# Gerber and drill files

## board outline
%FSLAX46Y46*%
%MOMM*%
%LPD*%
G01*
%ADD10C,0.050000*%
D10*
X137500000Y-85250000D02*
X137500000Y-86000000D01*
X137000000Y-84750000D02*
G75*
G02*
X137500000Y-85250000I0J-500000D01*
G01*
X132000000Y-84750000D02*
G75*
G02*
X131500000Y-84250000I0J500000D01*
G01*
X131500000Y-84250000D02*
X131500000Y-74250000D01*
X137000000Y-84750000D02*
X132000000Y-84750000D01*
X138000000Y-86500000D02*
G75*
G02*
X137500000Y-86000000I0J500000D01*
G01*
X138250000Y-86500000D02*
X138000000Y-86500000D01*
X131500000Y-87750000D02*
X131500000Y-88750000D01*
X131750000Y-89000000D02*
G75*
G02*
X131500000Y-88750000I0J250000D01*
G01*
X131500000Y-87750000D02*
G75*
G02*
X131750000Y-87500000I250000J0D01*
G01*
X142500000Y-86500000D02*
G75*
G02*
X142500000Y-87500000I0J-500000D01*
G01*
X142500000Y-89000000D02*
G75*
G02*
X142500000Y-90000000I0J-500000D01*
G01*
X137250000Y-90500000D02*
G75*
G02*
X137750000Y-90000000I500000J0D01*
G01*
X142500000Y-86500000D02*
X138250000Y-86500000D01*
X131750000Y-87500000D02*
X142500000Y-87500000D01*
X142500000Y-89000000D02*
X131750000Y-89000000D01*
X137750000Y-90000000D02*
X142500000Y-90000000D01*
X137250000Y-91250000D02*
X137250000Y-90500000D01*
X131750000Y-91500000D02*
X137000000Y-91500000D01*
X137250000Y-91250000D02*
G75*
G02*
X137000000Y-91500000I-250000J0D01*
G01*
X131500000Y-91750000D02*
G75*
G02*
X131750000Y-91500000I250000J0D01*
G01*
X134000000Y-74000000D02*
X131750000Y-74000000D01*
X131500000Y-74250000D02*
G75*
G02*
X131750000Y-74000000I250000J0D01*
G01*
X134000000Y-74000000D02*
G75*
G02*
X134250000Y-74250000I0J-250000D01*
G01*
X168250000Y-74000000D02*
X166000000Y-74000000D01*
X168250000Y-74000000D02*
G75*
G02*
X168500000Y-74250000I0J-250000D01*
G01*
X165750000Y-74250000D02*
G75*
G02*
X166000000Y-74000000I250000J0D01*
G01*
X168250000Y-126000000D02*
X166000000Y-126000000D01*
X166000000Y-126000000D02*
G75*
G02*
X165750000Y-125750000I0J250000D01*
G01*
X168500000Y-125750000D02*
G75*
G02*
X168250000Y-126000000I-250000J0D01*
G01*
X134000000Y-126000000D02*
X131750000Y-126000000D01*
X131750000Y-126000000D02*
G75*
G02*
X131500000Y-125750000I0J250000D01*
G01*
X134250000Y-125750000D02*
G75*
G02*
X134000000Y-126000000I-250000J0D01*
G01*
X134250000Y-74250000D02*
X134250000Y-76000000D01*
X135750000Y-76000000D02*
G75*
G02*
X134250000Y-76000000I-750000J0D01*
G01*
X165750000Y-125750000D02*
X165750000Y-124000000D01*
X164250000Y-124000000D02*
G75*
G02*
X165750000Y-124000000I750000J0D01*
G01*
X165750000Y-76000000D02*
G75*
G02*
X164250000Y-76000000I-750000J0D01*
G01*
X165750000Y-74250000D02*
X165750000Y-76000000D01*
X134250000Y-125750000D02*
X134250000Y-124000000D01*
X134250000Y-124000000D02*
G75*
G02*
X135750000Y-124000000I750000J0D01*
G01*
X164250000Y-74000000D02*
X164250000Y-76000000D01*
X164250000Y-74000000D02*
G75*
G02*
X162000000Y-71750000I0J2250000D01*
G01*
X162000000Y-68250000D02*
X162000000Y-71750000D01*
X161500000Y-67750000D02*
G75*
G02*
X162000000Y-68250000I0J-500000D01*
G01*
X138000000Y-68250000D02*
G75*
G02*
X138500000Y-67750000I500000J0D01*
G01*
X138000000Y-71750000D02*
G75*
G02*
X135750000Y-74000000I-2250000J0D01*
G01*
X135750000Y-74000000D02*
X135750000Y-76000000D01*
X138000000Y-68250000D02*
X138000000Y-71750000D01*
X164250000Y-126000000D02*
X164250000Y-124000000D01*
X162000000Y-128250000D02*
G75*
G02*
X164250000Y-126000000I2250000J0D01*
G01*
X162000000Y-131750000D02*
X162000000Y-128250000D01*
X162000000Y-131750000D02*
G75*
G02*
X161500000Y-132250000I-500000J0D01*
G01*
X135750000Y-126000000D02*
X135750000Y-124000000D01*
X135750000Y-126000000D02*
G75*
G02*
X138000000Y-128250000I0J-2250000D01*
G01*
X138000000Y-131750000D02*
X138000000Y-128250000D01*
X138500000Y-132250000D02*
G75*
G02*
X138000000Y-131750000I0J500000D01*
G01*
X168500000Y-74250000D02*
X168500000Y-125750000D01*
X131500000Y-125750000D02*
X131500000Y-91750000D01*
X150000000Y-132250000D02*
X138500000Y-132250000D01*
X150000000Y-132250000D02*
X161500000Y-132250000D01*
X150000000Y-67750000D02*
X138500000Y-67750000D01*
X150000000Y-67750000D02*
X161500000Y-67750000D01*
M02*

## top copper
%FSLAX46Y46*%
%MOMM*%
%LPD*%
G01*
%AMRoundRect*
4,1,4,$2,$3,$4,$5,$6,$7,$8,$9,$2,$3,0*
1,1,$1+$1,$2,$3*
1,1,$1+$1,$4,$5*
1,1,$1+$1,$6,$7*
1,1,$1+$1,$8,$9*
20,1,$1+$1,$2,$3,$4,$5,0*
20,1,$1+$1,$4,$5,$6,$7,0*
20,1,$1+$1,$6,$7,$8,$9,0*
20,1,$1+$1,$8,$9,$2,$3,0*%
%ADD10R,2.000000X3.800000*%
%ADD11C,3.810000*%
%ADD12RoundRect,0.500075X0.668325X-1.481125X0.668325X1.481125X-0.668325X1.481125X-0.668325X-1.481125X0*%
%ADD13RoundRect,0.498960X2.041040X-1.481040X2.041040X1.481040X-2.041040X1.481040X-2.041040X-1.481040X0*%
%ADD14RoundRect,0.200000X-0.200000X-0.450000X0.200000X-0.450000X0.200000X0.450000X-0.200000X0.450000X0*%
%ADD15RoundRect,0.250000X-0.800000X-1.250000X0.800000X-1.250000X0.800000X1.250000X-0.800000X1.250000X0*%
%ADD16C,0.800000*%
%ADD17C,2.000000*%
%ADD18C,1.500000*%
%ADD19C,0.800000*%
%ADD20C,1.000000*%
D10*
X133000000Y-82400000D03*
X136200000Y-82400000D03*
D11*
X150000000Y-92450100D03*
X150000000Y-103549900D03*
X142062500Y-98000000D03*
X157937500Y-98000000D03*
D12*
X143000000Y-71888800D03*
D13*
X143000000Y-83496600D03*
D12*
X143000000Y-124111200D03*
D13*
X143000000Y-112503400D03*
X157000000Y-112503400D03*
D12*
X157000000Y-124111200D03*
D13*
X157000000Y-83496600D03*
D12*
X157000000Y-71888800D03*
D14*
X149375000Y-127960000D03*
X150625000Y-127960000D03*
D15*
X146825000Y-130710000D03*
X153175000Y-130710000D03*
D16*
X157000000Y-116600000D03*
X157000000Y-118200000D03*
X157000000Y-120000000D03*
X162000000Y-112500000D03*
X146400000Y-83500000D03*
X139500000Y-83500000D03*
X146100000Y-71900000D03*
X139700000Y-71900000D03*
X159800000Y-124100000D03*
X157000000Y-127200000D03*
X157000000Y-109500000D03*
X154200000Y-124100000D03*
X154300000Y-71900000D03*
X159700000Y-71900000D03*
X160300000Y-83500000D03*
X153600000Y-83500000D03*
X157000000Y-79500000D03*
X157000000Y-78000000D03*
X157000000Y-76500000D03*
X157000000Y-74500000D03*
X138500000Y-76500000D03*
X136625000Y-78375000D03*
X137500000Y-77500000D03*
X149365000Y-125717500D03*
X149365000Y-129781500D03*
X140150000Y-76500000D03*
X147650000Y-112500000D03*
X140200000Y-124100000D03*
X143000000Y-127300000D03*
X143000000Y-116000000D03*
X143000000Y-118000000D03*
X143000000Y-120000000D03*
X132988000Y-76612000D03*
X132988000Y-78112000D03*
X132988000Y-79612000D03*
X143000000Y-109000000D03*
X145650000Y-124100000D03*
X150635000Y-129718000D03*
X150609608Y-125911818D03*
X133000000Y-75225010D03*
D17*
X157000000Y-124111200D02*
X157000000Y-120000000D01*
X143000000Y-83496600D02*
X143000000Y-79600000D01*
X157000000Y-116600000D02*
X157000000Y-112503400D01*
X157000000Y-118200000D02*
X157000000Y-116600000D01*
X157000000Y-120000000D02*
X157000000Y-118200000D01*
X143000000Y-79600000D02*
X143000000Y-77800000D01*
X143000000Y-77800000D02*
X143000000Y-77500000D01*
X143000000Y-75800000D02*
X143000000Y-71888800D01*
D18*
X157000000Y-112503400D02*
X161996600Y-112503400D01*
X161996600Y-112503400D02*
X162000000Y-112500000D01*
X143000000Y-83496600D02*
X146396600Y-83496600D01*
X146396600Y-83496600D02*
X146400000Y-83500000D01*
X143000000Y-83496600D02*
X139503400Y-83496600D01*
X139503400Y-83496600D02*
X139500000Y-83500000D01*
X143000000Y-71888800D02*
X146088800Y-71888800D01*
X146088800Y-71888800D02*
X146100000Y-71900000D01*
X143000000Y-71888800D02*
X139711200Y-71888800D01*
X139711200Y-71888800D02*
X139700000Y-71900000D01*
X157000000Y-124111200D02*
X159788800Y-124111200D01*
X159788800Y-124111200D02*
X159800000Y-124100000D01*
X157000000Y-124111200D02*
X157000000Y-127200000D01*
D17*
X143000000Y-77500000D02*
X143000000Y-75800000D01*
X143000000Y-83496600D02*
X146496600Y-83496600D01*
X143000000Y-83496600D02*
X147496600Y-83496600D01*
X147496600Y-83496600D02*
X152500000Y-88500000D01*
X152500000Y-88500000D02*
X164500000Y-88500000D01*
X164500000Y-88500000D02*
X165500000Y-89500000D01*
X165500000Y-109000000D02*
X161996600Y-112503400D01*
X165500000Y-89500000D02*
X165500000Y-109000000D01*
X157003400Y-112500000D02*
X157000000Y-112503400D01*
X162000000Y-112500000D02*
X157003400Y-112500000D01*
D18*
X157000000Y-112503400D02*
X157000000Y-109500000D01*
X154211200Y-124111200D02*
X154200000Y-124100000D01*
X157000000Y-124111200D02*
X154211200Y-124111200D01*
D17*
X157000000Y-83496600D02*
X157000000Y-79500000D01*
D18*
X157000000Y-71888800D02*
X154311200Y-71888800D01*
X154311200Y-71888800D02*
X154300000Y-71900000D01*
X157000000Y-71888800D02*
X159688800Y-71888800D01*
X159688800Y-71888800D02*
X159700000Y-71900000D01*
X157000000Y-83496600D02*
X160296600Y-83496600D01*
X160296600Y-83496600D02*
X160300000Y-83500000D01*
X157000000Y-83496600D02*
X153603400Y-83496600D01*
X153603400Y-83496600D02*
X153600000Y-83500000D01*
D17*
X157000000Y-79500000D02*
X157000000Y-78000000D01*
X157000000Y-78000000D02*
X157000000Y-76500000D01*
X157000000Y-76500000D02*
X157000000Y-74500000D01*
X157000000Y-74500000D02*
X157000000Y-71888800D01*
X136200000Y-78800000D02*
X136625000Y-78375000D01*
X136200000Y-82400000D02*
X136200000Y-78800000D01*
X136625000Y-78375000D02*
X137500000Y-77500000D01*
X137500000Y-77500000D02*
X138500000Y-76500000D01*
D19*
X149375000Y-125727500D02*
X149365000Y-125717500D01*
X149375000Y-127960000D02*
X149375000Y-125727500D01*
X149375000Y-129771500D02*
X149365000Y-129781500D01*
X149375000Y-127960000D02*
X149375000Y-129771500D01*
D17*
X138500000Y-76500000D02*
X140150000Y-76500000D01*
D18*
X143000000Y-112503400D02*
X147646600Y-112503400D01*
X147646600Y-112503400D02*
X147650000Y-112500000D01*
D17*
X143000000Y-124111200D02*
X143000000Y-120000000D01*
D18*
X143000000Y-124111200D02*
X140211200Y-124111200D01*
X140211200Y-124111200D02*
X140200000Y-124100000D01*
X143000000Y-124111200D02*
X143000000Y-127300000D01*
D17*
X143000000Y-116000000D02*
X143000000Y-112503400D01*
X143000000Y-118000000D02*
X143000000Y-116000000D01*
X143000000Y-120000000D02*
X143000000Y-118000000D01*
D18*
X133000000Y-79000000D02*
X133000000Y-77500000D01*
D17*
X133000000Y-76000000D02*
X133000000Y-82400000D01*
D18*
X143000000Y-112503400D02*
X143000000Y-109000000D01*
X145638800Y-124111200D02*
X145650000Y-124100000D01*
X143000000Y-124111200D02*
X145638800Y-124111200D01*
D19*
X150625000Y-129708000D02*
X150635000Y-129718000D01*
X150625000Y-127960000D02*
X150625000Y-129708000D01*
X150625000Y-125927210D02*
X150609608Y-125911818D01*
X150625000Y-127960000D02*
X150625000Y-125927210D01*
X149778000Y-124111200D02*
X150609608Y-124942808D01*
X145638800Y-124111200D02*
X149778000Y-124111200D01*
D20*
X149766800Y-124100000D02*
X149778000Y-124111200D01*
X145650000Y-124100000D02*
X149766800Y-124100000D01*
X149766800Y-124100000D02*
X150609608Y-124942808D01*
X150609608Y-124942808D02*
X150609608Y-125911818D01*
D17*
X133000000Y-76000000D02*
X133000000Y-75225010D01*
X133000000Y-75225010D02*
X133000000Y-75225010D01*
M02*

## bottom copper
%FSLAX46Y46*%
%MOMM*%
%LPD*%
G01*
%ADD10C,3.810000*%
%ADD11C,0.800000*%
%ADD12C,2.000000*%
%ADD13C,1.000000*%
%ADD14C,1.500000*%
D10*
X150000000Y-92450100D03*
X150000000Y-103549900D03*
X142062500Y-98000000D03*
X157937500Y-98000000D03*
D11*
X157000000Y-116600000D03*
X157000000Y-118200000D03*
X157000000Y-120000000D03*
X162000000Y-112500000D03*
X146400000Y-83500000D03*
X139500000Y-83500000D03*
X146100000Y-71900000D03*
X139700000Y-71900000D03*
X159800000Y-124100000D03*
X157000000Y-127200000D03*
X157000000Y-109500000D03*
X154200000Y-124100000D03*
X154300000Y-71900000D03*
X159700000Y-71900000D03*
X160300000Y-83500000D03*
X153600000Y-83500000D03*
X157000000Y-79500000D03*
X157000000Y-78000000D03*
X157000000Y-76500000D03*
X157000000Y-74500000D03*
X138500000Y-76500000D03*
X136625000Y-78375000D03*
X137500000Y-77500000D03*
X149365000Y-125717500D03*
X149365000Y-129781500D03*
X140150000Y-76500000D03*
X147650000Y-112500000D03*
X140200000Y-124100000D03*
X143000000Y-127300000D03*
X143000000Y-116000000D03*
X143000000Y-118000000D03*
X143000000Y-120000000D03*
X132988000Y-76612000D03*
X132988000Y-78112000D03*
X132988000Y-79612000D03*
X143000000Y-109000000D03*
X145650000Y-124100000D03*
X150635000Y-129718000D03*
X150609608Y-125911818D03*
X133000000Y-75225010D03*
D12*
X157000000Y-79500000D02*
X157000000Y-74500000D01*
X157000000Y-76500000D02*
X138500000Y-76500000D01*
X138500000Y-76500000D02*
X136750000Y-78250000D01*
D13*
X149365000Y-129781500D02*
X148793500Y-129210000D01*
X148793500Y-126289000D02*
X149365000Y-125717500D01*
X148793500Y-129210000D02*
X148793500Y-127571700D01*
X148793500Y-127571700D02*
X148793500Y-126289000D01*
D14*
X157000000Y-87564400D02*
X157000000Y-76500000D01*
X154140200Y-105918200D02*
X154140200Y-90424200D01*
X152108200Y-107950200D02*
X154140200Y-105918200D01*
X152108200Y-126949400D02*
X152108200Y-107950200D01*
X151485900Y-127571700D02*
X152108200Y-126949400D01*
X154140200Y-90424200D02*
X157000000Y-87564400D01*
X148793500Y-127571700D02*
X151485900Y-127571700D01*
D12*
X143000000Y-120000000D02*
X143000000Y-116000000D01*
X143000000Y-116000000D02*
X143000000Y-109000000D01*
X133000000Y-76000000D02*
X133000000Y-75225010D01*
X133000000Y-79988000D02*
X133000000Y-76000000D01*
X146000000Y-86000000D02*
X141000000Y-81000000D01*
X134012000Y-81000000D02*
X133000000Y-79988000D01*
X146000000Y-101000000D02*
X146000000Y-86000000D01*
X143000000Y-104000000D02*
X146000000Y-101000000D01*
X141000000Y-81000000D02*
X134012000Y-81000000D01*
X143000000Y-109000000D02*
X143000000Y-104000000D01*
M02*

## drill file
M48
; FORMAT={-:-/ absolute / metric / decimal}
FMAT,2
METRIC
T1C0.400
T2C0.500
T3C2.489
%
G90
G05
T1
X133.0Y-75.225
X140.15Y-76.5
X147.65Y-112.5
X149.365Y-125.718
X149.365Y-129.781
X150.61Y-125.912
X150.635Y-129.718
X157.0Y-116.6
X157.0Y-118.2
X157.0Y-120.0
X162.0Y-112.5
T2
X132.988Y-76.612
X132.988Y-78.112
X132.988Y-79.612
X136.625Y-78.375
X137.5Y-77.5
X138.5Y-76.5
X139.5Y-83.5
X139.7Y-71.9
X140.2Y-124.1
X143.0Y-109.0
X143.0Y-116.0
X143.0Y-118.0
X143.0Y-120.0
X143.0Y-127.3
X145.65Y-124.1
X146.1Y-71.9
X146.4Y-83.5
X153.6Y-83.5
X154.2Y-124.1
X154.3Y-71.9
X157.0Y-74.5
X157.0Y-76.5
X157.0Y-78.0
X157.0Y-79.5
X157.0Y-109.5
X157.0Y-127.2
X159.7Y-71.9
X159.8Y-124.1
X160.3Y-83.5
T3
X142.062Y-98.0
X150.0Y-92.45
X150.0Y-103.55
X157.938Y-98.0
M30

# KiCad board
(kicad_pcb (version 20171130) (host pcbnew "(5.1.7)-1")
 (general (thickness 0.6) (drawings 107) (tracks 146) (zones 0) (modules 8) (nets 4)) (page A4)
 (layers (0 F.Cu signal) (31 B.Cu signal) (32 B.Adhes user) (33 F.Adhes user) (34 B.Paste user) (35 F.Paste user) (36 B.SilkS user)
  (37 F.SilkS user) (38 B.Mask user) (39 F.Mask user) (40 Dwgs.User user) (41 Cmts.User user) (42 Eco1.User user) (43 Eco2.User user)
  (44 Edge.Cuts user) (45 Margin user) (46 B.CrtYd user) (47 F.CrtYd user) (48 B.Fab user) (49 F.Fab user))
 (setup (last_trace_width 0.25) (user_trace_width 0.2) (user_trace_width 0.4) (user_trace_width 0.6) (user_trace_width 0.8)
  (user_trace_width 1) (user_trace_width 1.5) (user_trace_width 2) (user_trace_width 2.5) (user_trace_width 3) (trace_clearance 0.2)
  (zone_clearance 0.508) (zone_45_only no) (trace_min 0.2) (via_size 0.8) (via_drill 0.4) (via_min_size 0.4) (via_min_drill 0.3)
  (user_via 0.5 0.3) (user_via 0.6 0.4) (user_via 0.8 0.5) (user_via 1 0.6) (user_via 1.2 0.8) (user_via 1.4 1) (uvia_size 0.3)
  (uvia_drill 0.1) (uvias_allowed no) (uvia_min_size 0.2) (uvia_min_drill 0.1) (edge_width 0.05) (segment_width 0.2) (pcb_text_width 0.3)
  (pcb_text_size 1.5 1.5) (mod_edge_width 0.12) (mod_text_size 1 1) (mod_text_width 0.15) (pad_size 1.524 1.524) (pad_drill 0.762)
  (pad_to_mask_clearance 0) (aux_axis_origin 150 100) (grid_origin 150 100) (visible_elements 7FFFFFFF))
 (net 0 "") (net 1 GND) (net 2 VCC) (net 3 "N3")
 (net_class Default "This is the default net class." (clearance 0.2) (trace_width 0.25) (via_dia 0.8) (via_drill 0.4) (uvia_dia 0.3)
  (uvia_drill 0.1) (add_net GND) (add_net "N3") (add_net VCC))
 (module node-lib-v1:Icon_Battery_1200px (layer F.Cu) (at 165.1 117.75)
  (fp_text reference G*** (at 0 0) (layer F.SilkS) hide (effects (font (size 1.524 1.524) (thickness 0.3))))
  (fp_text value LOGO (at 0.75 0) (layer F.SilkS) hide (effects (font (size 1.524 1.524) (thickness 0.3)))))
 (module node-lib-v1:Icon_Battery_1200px (layer F.Cu) (at 135.05 117.6)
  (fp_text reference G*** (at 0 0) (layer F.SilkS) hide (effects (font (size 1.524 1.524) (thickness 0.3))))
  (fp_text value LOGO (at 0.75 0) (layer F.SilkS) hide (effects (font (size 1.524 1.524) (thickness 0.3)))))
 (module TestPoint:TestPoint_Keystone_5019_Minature (layer F.Cu) (at 133 82.4 270)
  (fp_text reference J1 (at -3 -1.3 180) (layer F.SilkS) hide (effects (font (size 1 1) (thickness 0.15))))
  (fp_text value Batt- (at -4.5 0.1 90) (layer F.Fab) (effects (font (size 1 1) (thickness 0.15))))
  (pad 1 smd rect (at 0 0 270) (size 3.8 2) (layers F.Cu F.Paste F.Mask) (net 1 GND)))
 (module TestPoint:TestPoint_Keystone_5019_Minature (layer F.Cu) (at 136.2 82.4 90)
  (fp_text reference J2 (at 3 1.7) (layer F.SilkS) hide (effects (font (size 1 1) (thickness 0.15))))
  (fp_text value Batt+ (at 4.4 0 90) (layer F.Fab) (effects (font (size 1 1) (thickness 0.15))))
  (pad 1 smd rect (at 0 0 90) (size 3.8 2) (layers F.Cu F.Paste F.Mask) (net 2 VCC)))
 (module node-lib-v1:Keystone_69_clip (layer F.Cu) (at 150 98 180)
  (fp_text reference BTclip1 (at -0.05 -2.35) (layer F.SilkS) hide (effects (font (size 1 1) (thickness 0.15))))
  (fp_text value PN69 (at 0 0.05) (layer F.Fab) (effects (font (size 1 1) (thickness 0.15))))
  (pad 2 smd circle (at 7.9375 0 180) (size 3.81 3.81) (layers F.Paste F.Mask))
  (pad 2 smd circle (at -7.9375 0 180) (size 3.81 3.81) (layers F.Paste F.Mask))
  (pad 2 smd circle (at 0 -5.5499 180) (size 3.81 3.81) (layers F.Paste F.Mask))
  (pad 2 smd circle (at 0 5.5499 180) (size 3.81 3.81) (layers F.Paste F.Mask))
  (pad 1 thru_hole circle (at 0 5.5499 180) (size 3.81 3.81) (drill 2.4892) (layers *.Cu *.Mask))
  (pad 1 thru_hole circle (at 0 -5.5499 180) (size 3.81 3.81) (drill 2.4892) (layers *.Cu *.Mask))
  (pad 1 thru_hole circle (at 7.9375 0 180) (size 3.81 3.81) (drill 2.4892) (layers *.Cu *.Mask))
  (pad 1 thru_hole circle (at -7.9375 0 180) (size 3.81 3.81) (drill 2.4892) (layers *.Cu *.Mask F.Paste)))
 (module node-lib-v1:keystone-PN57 (layer F.Cu) (at 143 98 90)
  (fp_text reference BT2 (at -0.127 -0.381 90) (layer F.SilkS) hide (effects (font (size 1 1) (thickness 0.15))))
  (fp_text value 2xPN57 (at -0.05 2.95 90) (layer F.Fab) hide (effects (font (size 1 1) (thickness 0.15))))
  (pad 1 smd roundrect (at 26.1112 0 90) (size 3.9624 2.3368) (layers F.Cu F.Paste F.Mask) (roundrect_rratio 0.2139999144128723)
   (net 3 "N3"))
  (pad 1 smd roundrect (at 14.5034 0 90) (size 3.96 5.08) (layers F.Cu F.Paste F.Mask) (roundrect_rratio 0.126) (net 3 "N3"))
  (pad 2 smd roundrect (at -26.1112 0 90) (size 3.9624 2.3368) (layers F.Cu F.Paste F.Mask) (roundrect_rratio 0.2139999144128723)
   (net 1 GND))
  (pad 2 smd roundrect (at -14.5034 0 90) (size 3.96 5.08) (layers F.Cu F.Paste F.Mask) (roundrect_rratio 0.126) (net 1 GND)))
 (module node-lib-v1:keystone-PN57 (layer F.Cu) (at 157 98 90)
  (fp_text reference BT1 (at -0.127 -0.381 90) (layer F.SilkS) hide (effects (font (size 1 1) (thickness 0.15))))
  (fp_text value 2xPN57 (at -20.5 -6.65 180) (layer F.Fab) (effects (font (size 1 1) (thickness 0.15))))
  (pad 2 smd roundrect (at -14.5034 0 90) (size 3.96 5.08) (layers F.Cu F.Paste F.Mask) (roundrect_rratio 0.126) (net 3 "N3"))
  (pad 2 smd roundrect (at -26.1112 0 90) (size 3.9624 2.3368) (layers F.Cu F.Paste F.Mask) (roundrect_rratio 0.2139999144128723)
   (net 3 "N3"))
  (pad 1 smd roundrect (at 14.5034 0 90) (size 3.96 5.08) (layers F.Cu F.Paste F.Mask) (roundrect_rratio 0.126) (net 2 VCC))
  (pad 1 smd roundrect (at 26.1112 0 90) (size 3.9624 2.3368) (layers F.Cu F.Paste F.Mask) (roundrect_rratio 0.2139999144128723) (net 2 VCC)))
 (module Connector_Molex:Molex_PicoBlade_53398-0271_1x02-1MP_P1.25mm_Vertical (layer F.Cu) (at 150 129.21)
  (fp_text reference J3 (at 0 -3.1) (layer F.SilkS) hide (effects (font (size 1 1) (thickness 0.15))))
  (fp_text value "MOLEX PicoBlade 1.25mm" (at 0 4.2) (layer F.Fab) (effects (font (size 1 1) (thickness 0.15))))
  (pad 1 smd roundrect (at -0.625 -1.25) (size 0.8 1.3) (layers F.Cu F.Paste F.Mask) (roundrect_rratio 0.25) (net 2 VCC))
  (pad 2 smd roundrect (at 0.625 -1.25) (size 0.8 1.3) (layers F.Cu F.Paste F.Mask) (roundrect_rratio 0.25) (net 1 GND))
  (pad MP smd roundrect (at -3.175 1.5) (size 2.1 3) (layers F.Cu F.Paste F.Mask) (roundrect_rratio 0.119047619047619))
  (pad MP smd roundrect (at 3.175 1.5) (size 2.1 3) (layers F.Cu F.Paste F.Mask) (roundrect_rratio 0.119047619047619)))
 (gr_line (start 137.5 85.25) (end 137.5 86) (layer Edge.Cuts) (width 0.05))
 (gr_arc (start 137 85.25) (end 137.5 85.25) (angle -90) (layer Edge.Cuts) (width 0.05))
 (gr_arc (start 132 84.25) (end 131.5 84.25) (angle -90) (layer Edge.Cuts) (width 0.05))
 (gr_line (start 131.5 84.25) (end 131.5 74.25) (layer Edge.Cuts) (width 0.05))
 (gr_line (start 137 84.75) (end 132 84.75) (layer Edge.Cuts) (width 0.05))
 (gr_arc (start 138 86) (end 137.5 86) (angle -90) (layer Edge.Cuts) (width 0.05))
 (gr_line (start 138.25 86.5) (end 138 86.5) (layer Edge.Cuts) (width 0.05))
 (gr_line (start 131.5 87.75) (end 131.5 88.75) (layer Edge.Cuts) (width 0.05))
 (gr_arc (start 131.75 88.75) (end 131.5 88.75) (angle -90) (layer Edge.Cuts) (width 0.05))
 (gr_arc (start 131.75 87.75) (end 131.75 87.5) (angle -90) (layer Edge.Cuts) (width 0.05))
 (gr_arc (start 142.5 87) (end 142.5 87.5) (angle -180) (layer Edge.Cuts) (width 0.05))
 (gr_arc (start 142.5 89.5) (end 142.5 90) (angle -180) (layer Edge.Cuts) (width 0.05))
 (gr_arc (start 137.75 90.5) (end 137.75 90) (angle -90) (layer Edge.Cuts) (width 0.05))
 (gr_line (start 142.5 86.5) (end 138.25 86.5) (layer Edge.Cuts) (width 0.05))
 (gr_line (start 131.75 87.5) (end 142.5 87.5) (layer Edge.Cuts) (width 0.05))
 (gr_line (start 142.5 89) (end 131.75 89) (layer Edge.Cuts) (width 0.05))
 (gr_line (start 137.75 90) (end 142.5 90) (layer Edge.Cuts) (width 0.05))
 (gr_line (start 137.25 91.25) (end 137.25 90.5) (layer Edge.Cuts) (width 0.05))
 (gr_line (start 131.75 91.5) (end 137 91.5) (layer Edge.Cuts) (width 0.05))
 (gr_arc (start 137 91.25) (end 137 91.5) (angle -90) (layer Edge.Cuts) (width 0.05))
 (gr_arc (start 131.75 91.75) (end 131.75 91.5) (angle -90) (layer Edge.Cuts) (width 0.05))
 (gr_line (start 134 74) (end 131.75 74) (layer Edge.Cuts) (width 0.05))
 (gr_arc (start 131.75 74.25) (end 131.75 74) (angle -90) (layer Edge.Cuts) (width 0.05))
 (gr_arc (start 134 74.25) (end 134.25 74.25) (angle -90) (layer Edge.Cuts) (width 0.05))
 (gr_line (start 168.25 74) (end 166 74) (layer Edge.Cuts) (width 0.05))
 (gr_arc (start 168.25 74.25) (end 168.5 74.25) (angle -90) (layer Edge.Cuts) (width 0.05))
 (gr_arc (start 166 74.25) (end 166 74) (angle -90) (layer Edge.Cuts) (width 0.05))
 (gr_line (start 168.25 126) (end 166 126) (layer Edge.Cuts) (width 0.05))
 (gr_arc (start 166 125.75) (end 165.75 125.75) (angle -90) (layer Edge.Cuts) (width 0.05))
 (gr_arc (start 168.25 125.75) (end 168.25 126) (angle -90) (layer Edge.Cuts) (width 0.05))
 (gr_line (start 134 126) (end 131.75 126) (layer Edge.Cuts) (width 0.05))
 (gr_arc (start 131.75 125.75) (end 131.5 125.75) (angle -90) (layer Edge.Cuts) (width 0.05))
 (gr_arc (start 134 125.75) (end 134 126) (angle -90) (layer Edge.Cuts) (width 0.05))
 (gr_line (start 134.25 74.25) (end 134.25 76) (layer Edge.Cuts) (width 0.05))
 (gr_arc (start 135 76) (end 134.25 76) (angle -180) (layer Edge.Cuts) (width 0.05))
 (gr_line (start 165.75 125.75) (end 165.75 124) (layer Edge.Cuts) (width 0.05))
 (gr_arc (start 165 124) (end 165.75 124) (angle -180) (layer Edge.Cuts) (width 0.05))
 (gr_arc (start 165 76) (end 164.25 76) (angle -180) (layer Edge.Cuts) (width 0.05))
 (gr_line (start 165.75 74.25) (end 165.75 76) (layer Edge.Cuts) (width 0.05))
 (gr_line (start 134.25 125.75) (end 134.25 124) (layer Edge.Cuts) (width 0.05))
 (gr_arc (start 135 124) (end 135.75 124) (angle -180) (layer Edge.Cuts) (width 0.05))
 (gr_line (start 164.25 74) (end 164.25 76) (layer Edge.Cuts) (width 0.05))
 (gr_arc (start 164.25 71.75) (end 162 71.75) (angle -90) (layer Edge.Cuts) (width 0.05))
 (gr_line (start 162 68.25) (end 162 71.75) (layer Edge.Cuts) (width 0.05))
 (gr_arc (start 161.5 68.25) (end 162 68.25) (angle -90) (layer Edge.Cuts) (width 0.05))
 (gr_arc (start 138.5 68.25) (end 138.5 67.75) (angle -90) (layer Edge.Cuts) (width 0.05))
 (gr_arc (start 135.75 71.75) (end 135.75 74) (angle -90) (layer Edge.Cuts) (width 0.05))
 (gr_line (start 135.75 74) (end 135.75 76) (layer Edge.Cuts) (width 0.05))
 (gr_line (start 138 68.25) (end 138 71.75) (layer Edge.Cuts) (width 0.05))
 (gr_line (start 164.25 126) (end 164.25 124) (layer Edge.Cuts) (width 0.05))
 (gr_arc (start 164.25 128.25) (end 164.25 126) (angle -90) (layer Edge.Cuts) (width 0.05))
 (gr_line (start 162 131.75) (end 162 128.25) (layer Edge.Cuts) (width 0.05))
 (gr_arc (start 161.5 131.75) (end 161.5 132.25) (angle -90) (layer Edge.Cuts) (width 0.05))
 (gr_line (start 135.75 126) (end 135.75 124) (layer Edge.Cuts) (width 0.05))
 (gr_arc (start 135.75 128.25) (end 138 128.25) (angle -90) (layer Edge.Cuts) (width 0.05))
 (gr_line (start 138 131.75) (end 138 128.25) (layer Edge.Cuts) (width 0.05))
 (gr_arc (start 138.5 131.75) (end 138 131.75) (angle -90) (layer Edge.Cuts) (width 0.05))
 (gr_line (start 168.5 74.25) (end 168.5 125.75) (layer Edge.Cuts) (width 0.05))
 (gr_line (start 131.5 125.75) (end 131.5 91.75) (layer Edge.Cuts) (width 0.05))
 (gr_line (start 150 132.25) (end 138.5 132.25) (layer Edge.Cuts) (width 0.05))
 (gr_line (start 150 132.25) (end 161.5 132.25) (layer Edge.Cuts) (width 0.05))
 (gr_line (start 150 67.75) (end 138.5 67.75) (layer Edge.Cuts) (width 0.05))
 (gr_line (start 150 67.75) (end 161.5 67.75) (layer Edge.Cuts) (width 0.05))
 (segment (start 157 124.1112) (end 157 120) (width 2) (layer F.Cu) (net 3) (status 10))
 (segment (start 143 83.4966) (end 143 79.6) (width 2) (layer F.Cu) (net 3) (status 10))
 (segment (start 157 116.6) (end 157 112.5034) (width 2) (layer F.Cu) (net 3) (status 20))
 (via (at 157 116.6) (size 0.8) (drill 0.4) (layers F.Cu B.Cu) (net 3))
 (segment (start 157 118.2) (end 157 116.6) (width 2) (layer F.Cu) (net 3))
 (via (at 157 118.2) (size 0.8) (drill 0.4) (layers F.Cu B.Cu) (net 3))
 (segment (start 157 120) (end 157 118.2) (width 2) (layer F.Cu) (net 3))
 (via (at 157 120) (size 0.8) (drill 0.4) (layers F.Cu B.Cu) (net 3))
 (segment (start 143 79.6) (end 143 77.8) (width 2) (layer F.Cu) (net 3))
 (segment (start 143 77.8) (end 143 77.5) (width 2) (layer F.Cu) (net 3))
 (segment (start 143 75.8) (end 143 71.8888) (width 2) (layer F.Cu) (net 3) (status 20))
 (via (at 162 112.5) (size 0.8) (drill 0.4) (layers F.Cu B.Cu) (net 3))
 (segment (start 157 112.5034) (end 161.9966 112.5034) (width 1.5) (layer F.Cu) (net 3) (status 10))
 (segment (start 161.9966 112.5034) (end 162 112.5) (width 1.5) (layer F.Cu) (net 3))
 (via (at 146.4 83.5) (size 0.8) (drill 0.5) (layers F.Cu B.Cu) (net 3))
 (segment (start 143 83.4966) (end 146.3966 83.4966) (width 1.5) (layer F.Cu) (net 3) (status 10))
 (segment (start 146.3966 83.4966) (end 146.4 83.5) (width 1.5) (layer F.Cu) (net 3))
 (via (at 139.5 83.5) (size 0.8) (drill 0.5) (layers F.Cu B.Cu) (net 3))
 (segment (start 143 83.4966) (end 139.5034 83.4966) (width 1.5) (layer F.Cu) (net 3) (status 10))
 (segment (start 139.5034 83.4966) (end 139.5 83.5) (width 1.5) (layer F.Cu) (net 3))
 (via (at 146.1 71.9) (size 0.8) (drill 0.5) (layers F.Cu B.Cu) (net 3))
 (segment (start 143 71.8888) (end 146.0888 71.8888) (width 1.5) (layer F.Cu) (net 3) (status 10))
 (segment (start 146.0888 71.8888) (end 146.1 71.9) (width 1.5) (layer F.Cu) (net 3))
 (via (at 139.7 71.9) (size 0.8) (drill 0.5) (layers F.Cu B.Cu) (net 3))
 (segment (start 143 71.8888) (end 139.7112 71.8888) (width 1.5) (layer F.Cu) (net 3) (status 10))
 (segment (start 139.7112 71.8888) (end 139.7 71.9) (width 1.5) (layer F.Cu) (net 3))
 (via (at 159.8 124.1) (size 0.8) (drill 0.5) (layers F.Cu B.Cu) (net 3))
 (segment (start 157 124.1112) (end 159.7888 124.1112) (width 1.5) (layer F.Cu) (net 3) (status 10))
 (segment (start 159.7888 124.1112) (end 159.8 124.1) (width 1.5) (layer F.Cu) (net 3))
 (via (at 157 127.2) (size 0.8) (drill 0.5) (layers F.Cu B.Cu) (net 3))
 (segment (start 157 124.1112) (end 157 127.2) (width 1.5) (layer F.Cu) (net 3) (status 10))
 (segment (start 143 77.5) (end 143 75.8) (width 2) (layer F.Cu) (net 3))
 (segment (start 143 83.4966) (end 146.4966 83.4966) (width 2) (layer F.Cu) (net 3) (status 10))
 (segment (start 143 83.4966) (end 147.4966 83.4966) (width 2) (layer F.Cu) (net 3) (status 10))
 (segment (start 147.4966 83.4966) (end 152.5 88.5) (width 2) (layer F.Cu) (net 3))
 (segment (start 152.5 88.5) (end 164.5 88.5) (width 2) (layer F.Cu) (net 3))
 (segment (start 164.5 88.5) (end 165.5 89.5) (width 2) (layer F.Cu) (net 3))
 (segment (start 165.5 109) (end 161.9966 112.5034) (width 2) (layer F.Cu) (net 3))
 (segment (start 165.5 89.5) (end 165.5 109) (width 2) (layer F.Cu) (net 3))
 (segment (start 157.0034 112.5) (end 157 112.5034) (width 2) (layer F.Cu) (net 3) (status 30))
 (segment (start 162 112.5) (end 157.0034 112.5) (width 2) (layer F.Cu) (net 3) (status 20))
 (segment (start 157 112.5034) (end 157 109.5) (width 1.5) (layer F.Cu) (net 3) (status 10))
 (via (at 157 109.5) (size 0.8) (drill 0.5) (layers F.Cu B.Cu) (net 3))
 (via (at 154.2 124.1) (size 0.8) (drill 0.5) (layers F.Cu B.Cu) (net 3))
 (segment (start 154.2112 124.1112) (end 154.2 124.1) (width 1.5) (layer F.Cu) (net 3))
 (segment (start 157 124.1112) (end 154.2112 124.1112) (width 1.5) (layer F.Cu) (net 3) (status 10))
 (segment (start 157 83.4966) (end 157 79.5) (width 2) (layer F.Cu) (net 2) (status 10))
 (via (at 154.3 71.9) (size 0.8) (drill 0.5) (layers F.Cu B.Cu) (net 2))
 (segment (start 157 71.8888) (end 154.3112 71.8888) (width 1.5) (layer F.Cu) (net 2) (status 10))
 (segment (start 154.3112 71.8888) (end 154.3 71.9) (width 1.5) (layer F.Cu) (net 2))
 (segment (start 157 71.8888) (end 159.6888 71.8888) (width 1.5) (layer F.Cu) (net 2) (status 10))
 (via (at 159.7 71.9) (size 0.8) (drill 0.5) (layers F.Cu B.Cu) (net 2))
 (segment (start 159.6888 71.8888) (end 159.7 71.9) (width 1.5) (layer F.Cu) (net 2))
 (via (at 160.3 83.5) (size 0.8) (drill 0.5) (layers F.Cu B.Cu) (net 2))
 (segment (start 157 83.4966) (end 160.2966 83.4966) (width 1.5) (layer F.Cu) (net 2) (status 10))
 (segment (start 160.2966 83.4966) (end 160.3 83.5) (width 1.5) (layer F.Cu) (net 2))
 (via (at 153.6 83.5) (size 0.8) (drill 0.5) (layers F.Cu B.Cu) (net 2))
 (segment (start 157 83.4966) (end 153.6034 83.4966) (width 1.5) (layer F.Cu) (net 2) (status 10))
 (segment (start 153.6034 83.4966) (end 153.6 83.5) (width 1.5) (layer F.Cu) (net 2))
 (segment (start 157 79.5) (end 157 78) (width 2) (layer F.Cu) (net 2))
 (via (at 157 79.5) (size 0.8) (drill 0.5) (layers F.Cu B.Cu) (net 2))
 (segment (start 157 78) (end 157 76.5) (width 2) (layer F.Cu) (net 2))
 (via (at 157 78) (size 0.8) (drill 0.5) (layers F.Cu B.Cu) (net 2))
 (segment (start 157 76.5) (end 157 74.5) (width 2) (layer F.Cu) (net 2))
 (via (at 157 76.5) (size 0.8) (drill 0.5) (layers F.Cu B.Cu) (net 2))
 (segment (start 157 74.5) (end 157 71.8888) (width 2) (layer F.Cu) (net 2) (status 20))
 (via (at 157 74.5) (size 0.8) (drill 0.5) (layers F.Cu B.Cu) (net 2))
 (segment (start 157 79.5) (end 157 74.5) (width 2) (layer B.Cu) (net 2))
 (segment (start 157 76.5) (end 138.5 76.5) (width 2) (layer B.Cu) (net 2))
 (segment (start 138.5 76.5) (end 136.75 78.25) (width 2) (layer B.Cu) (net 2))
 (via (at 138.5 76.5) (size 0.8) (drill 0.5) (layers F.Cu B.Cu) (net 2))
 (segment (start 136.2 78.8) (end 136.625 78.375) (width 2) (layer F.Cu) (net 2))
 (segment (start 136.2 82.4) (end 136.2 78.8) (width 2) (layer F.Cu) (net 2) (status 10))
 (segment (start 136.625 78.375) (end 137.5 77.5) (width 2) (layer F.Cu) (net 2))
 (via (at 136.625 78.375) (size 0.8) (drill 0.5) (layers F.Cu B.Cu) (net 2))
 (segment (start 137.5 77.5) (end 138.5 76.5) (width 2) (layer F.Cu) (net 2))
 (via (at 137.5 77.5) (size 0.8) (drill 0.5) (layers F.Cu B.Cu) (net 2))
 (via (at 149.365 125.7175) (size 0.8) (drill 0.4) (layers F.Cu B.Cu) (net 2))
 (segment (start 149.375 125.7275) (end 149.365 125.7175) (width 0.8) (layer F.Cu) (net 2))
 (segment (start 149.375 127.96) (end 149.375 125.7275) (width 0.8) (layer F.Cu) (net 2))
 (via (at 149.365 129.7815) (size 0.8) (drill 0.4) (layers F.Cu B.Cu) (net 2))
 (segment (start 149.375 129.7715) (end 149.365 129.7815) (width 0.8) (layer F.Cu) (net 2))
 (segment (start 149.375 127.96) (end 149.375 129.7715) (width 0.8) (layer F.Cu) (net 2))
 (segment (start 149.365 129.7815) (end 148.7935 129.21) (width 1) (layer B.Cu) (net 2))
 (segment (start 148.7935 126.289) (end 149.365 125.7175) (width 1) (layer B.Cu) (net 2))
 (segment (start 148.7935 129.21) (end 148.7935 127.5717) (width 1) (layer B.Cu) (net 2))
 (segment (start 148.7935 127.5717) (end 148.7935 126.289) (width 1) (layer B.Cu) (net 2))
 (segment (start 157 87.5644) (end 157 76.5) (width 1.5) (layer B.Cu) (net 2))
 (segment (start 154.1402 105.9182) (end 154.1402 90.4242) (width 1.5) (layer B.Cu) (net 2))
 (segment (start 152.1082 107.9502) (end 154.1402 105.9182) (width 1.5) (layer B.Cu) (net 2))
 (segment (start 152.1082 126.9494) (end 152.1082 107.9502) (width 1.5) (layer B.Cu) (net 2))
 (segment (start 151.4859 127.5717) (end 152.1082 126.9494) (width 1.5) (layer B.Cu) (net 2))
 (segment (start 154.1402 90.4242) (end 157 87.5644) (width 1.5) (layer B.Cu) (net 2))
 (segment (start 148.7935 127.5717) (end 151.4859 127.5717) (width 1.5) (layer B.Cu) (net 2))
 (via (at 140.15 76.5) (size 0.8) (drill 0.4) (layers F.Cu B.Cu) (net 2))
 (segment (start 138.5 76.5) (end 140.15 76.5) (width 2) (layer F.Cu) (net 2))
 (via (at 147.65 112.5) (size 0.8) (drill 0.4) (layers F.Cu B.Cu) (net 1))
 (segment (start 143 112.5034) (end 147.6466 112.5034) (width 1.5) (layer F.Cu) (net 1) (status 10))
 (segment (start 147.6466 112.5034) (end 147.65 112.5) (width 1.5) (layer F.Cu) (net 1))
 (segment (start 143 124.1112) (end 143 120) (width 2) (layer F.Cu) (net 1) (status 10))
 (via (at 140.2 124.1) (size 0.8) (drill 0.5) (layers F.Cu B.Cu) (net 1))
 (segment (start 143 124.1112) (end 140.2112 124.1112) (width 1.5) (layer F.Cu) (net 1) (status 10))
 (segment (start 140.2112 124.1112) (end 140.2 124.1) (width 1.5) (layer F.Cu) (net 1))
 (via (at 143 127.3) (size 0.8) (drill 0.5) (layers F.Cu B.Cu) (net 1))
 (segment (start 143 124.1112) (end 143 127.3) (width 1.5) (layer F.Cu) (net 1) (status 10))
 (segment (start 143 116) (end 143 112.5034) (width 2) (layer F.Cu) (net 1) (status 20))
 (via (at 143 116) (size 0.8) (drill 0.5) (layers F.Cu B.Cu) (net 1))
 (segment (start 143 118) (end 143 116) (width 2) (layer F.Cu) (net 1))
 (via (at 143 118) (size 0.8) (drill 0.5) (layers F.Cu B.Cu) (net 1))
 (segment (start 143 120) (end 143 118) (width 2) (layer F.Cu) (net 1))
 (via (at 143 120) (size 0.8) (drill 0.5) (layers F.Cu B.Cu) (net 1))
 (segment (start 143 120) (end 143 116) (width 2) (layer B.Cu) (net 1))
 (via (at 132.988 76.612) (size 0.8) (drill 0.5) (layers F.Cu B.Cu) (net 1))
 (via (at 132.988 78.112) (size 0.8) (drill 0.5) (layers F.Cu B.Cu) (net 1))
 (segment (start 133 79) (end 133 77.5) (width 1.5) (layer F.Cu) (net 1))
 (via (at 132.988 79.612) (size 0.8) (drill 0.5) (layers F.Cu B.Cu) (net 1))
 (segment (start 133 76) (end 133 82.4) (width 2) (layer F.Cu) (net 1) (status 20))
 (segment (start 143 116) (end 143 109) (width 2) (layer B.Cu) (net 1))
 (segment (start 143 112.5034) (end 143 109) (width 1.5) (layer F.Cu) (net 1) (status 10))
 (via (at 143 109) (size 0.8) (drill 0.5) (layers F.Cu B.Cu) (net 1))
 (segment (start 145.6388 124.1112) (end 145.65 124.1) (width 1.5) (layer F.Cu) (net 1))
 (via (at 145.65 124.1) (size 0.8) (drill 0.5) (layers F.Cu B.Cu) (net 1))
 (segment (start 143 124.1112) (end 145.6388 124.1112) (width 1.5) (layer F.Cu) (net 1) (status 10))
 (via (at 150.635 129.718) (size 0.8) (drill 0.4) (layers F.Cu B.Cu) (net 1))
 (segment (start 150.625 129.708) (end 150.635 129.718) (width 0.8) (layer F.Cu) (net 1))
 (segment (start 150.625 127.96) (end 150.625 129.708) (width 0.8) (layer F.Cu) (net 1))
 (via (at 150.609608 125.911818) (size 0.8) (drill 0.4) (layers F.Cu B.Cu) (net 1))
 (segment (start 150.625 125.92721) (end 150.609608 125.911818) (width 0.8) (layer F.Cu) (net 1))
 (segment (start 150.625 127.96) (end 150.625 125.92721) (width 0.8) (layer F.Cu) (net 1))
 (segment (start 149.778 124.1112) (end 150.609608 124.942808) (width 0.8) (layer F.Cu) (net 1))
 (segment (start 145.6388 124.1112) (end 149.778 124.1112) (width 0.8) (layer F.Cu) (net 1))
 (segment (start 149.7668 124.1) (end 149.778 124.1112) (width 1) (layer F.Cu) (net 1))
 (segment (start 145.65 124.1) (end 149.7668 124.1) (width 1) (layer F.Cu) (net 1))
 (segment (start 149.7668 124.1) (end 150.609608 124.942808) (width 1) (layer F.Cu) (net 1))
 (segment (start 150.609608 124.942808) (end 150.609608 125.911818) (width 1) (layer F.Cu) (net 1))
 (segment (start 133 76) (end 133 75.22501) (width 2) (layer F.Cu) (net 1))
 (segment (start 133 75.22501) (end 133 75.22501) (width 2) (layer F.Cu) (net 1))
 (via (at 133 75.22501) (size 0.8) (drill 0.4) (layers F.Cu B.Cu) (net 1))
 (segment (start 133 76) (end 133 75.22501) (width 2) (layer B.Cu) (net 1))
 (segment (start 133 79.988) (end 133 76) (width 2) (layer B.Cu) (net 1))
 (segment (start 146 86) (end 141 81) (width 2) (layer B.Cu) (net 1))
 (segment (start 134.012 81) (end 133 79.988) (width 2) (layer B.Cu) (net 1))
 (segment (start 146 101) (end 146 86) (width 2) (layer B.Cu) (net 1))
 (segment (start 143 104) (end 146 101) (width 2) (layer B.Cu) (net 1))
 (segment (start 141 81) (end 134.012 81) (width 2) (layer B.Cu) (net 1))
 (segment (start 143 109) (end 143 104) (width 2) (layer B.Cu) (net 1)))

